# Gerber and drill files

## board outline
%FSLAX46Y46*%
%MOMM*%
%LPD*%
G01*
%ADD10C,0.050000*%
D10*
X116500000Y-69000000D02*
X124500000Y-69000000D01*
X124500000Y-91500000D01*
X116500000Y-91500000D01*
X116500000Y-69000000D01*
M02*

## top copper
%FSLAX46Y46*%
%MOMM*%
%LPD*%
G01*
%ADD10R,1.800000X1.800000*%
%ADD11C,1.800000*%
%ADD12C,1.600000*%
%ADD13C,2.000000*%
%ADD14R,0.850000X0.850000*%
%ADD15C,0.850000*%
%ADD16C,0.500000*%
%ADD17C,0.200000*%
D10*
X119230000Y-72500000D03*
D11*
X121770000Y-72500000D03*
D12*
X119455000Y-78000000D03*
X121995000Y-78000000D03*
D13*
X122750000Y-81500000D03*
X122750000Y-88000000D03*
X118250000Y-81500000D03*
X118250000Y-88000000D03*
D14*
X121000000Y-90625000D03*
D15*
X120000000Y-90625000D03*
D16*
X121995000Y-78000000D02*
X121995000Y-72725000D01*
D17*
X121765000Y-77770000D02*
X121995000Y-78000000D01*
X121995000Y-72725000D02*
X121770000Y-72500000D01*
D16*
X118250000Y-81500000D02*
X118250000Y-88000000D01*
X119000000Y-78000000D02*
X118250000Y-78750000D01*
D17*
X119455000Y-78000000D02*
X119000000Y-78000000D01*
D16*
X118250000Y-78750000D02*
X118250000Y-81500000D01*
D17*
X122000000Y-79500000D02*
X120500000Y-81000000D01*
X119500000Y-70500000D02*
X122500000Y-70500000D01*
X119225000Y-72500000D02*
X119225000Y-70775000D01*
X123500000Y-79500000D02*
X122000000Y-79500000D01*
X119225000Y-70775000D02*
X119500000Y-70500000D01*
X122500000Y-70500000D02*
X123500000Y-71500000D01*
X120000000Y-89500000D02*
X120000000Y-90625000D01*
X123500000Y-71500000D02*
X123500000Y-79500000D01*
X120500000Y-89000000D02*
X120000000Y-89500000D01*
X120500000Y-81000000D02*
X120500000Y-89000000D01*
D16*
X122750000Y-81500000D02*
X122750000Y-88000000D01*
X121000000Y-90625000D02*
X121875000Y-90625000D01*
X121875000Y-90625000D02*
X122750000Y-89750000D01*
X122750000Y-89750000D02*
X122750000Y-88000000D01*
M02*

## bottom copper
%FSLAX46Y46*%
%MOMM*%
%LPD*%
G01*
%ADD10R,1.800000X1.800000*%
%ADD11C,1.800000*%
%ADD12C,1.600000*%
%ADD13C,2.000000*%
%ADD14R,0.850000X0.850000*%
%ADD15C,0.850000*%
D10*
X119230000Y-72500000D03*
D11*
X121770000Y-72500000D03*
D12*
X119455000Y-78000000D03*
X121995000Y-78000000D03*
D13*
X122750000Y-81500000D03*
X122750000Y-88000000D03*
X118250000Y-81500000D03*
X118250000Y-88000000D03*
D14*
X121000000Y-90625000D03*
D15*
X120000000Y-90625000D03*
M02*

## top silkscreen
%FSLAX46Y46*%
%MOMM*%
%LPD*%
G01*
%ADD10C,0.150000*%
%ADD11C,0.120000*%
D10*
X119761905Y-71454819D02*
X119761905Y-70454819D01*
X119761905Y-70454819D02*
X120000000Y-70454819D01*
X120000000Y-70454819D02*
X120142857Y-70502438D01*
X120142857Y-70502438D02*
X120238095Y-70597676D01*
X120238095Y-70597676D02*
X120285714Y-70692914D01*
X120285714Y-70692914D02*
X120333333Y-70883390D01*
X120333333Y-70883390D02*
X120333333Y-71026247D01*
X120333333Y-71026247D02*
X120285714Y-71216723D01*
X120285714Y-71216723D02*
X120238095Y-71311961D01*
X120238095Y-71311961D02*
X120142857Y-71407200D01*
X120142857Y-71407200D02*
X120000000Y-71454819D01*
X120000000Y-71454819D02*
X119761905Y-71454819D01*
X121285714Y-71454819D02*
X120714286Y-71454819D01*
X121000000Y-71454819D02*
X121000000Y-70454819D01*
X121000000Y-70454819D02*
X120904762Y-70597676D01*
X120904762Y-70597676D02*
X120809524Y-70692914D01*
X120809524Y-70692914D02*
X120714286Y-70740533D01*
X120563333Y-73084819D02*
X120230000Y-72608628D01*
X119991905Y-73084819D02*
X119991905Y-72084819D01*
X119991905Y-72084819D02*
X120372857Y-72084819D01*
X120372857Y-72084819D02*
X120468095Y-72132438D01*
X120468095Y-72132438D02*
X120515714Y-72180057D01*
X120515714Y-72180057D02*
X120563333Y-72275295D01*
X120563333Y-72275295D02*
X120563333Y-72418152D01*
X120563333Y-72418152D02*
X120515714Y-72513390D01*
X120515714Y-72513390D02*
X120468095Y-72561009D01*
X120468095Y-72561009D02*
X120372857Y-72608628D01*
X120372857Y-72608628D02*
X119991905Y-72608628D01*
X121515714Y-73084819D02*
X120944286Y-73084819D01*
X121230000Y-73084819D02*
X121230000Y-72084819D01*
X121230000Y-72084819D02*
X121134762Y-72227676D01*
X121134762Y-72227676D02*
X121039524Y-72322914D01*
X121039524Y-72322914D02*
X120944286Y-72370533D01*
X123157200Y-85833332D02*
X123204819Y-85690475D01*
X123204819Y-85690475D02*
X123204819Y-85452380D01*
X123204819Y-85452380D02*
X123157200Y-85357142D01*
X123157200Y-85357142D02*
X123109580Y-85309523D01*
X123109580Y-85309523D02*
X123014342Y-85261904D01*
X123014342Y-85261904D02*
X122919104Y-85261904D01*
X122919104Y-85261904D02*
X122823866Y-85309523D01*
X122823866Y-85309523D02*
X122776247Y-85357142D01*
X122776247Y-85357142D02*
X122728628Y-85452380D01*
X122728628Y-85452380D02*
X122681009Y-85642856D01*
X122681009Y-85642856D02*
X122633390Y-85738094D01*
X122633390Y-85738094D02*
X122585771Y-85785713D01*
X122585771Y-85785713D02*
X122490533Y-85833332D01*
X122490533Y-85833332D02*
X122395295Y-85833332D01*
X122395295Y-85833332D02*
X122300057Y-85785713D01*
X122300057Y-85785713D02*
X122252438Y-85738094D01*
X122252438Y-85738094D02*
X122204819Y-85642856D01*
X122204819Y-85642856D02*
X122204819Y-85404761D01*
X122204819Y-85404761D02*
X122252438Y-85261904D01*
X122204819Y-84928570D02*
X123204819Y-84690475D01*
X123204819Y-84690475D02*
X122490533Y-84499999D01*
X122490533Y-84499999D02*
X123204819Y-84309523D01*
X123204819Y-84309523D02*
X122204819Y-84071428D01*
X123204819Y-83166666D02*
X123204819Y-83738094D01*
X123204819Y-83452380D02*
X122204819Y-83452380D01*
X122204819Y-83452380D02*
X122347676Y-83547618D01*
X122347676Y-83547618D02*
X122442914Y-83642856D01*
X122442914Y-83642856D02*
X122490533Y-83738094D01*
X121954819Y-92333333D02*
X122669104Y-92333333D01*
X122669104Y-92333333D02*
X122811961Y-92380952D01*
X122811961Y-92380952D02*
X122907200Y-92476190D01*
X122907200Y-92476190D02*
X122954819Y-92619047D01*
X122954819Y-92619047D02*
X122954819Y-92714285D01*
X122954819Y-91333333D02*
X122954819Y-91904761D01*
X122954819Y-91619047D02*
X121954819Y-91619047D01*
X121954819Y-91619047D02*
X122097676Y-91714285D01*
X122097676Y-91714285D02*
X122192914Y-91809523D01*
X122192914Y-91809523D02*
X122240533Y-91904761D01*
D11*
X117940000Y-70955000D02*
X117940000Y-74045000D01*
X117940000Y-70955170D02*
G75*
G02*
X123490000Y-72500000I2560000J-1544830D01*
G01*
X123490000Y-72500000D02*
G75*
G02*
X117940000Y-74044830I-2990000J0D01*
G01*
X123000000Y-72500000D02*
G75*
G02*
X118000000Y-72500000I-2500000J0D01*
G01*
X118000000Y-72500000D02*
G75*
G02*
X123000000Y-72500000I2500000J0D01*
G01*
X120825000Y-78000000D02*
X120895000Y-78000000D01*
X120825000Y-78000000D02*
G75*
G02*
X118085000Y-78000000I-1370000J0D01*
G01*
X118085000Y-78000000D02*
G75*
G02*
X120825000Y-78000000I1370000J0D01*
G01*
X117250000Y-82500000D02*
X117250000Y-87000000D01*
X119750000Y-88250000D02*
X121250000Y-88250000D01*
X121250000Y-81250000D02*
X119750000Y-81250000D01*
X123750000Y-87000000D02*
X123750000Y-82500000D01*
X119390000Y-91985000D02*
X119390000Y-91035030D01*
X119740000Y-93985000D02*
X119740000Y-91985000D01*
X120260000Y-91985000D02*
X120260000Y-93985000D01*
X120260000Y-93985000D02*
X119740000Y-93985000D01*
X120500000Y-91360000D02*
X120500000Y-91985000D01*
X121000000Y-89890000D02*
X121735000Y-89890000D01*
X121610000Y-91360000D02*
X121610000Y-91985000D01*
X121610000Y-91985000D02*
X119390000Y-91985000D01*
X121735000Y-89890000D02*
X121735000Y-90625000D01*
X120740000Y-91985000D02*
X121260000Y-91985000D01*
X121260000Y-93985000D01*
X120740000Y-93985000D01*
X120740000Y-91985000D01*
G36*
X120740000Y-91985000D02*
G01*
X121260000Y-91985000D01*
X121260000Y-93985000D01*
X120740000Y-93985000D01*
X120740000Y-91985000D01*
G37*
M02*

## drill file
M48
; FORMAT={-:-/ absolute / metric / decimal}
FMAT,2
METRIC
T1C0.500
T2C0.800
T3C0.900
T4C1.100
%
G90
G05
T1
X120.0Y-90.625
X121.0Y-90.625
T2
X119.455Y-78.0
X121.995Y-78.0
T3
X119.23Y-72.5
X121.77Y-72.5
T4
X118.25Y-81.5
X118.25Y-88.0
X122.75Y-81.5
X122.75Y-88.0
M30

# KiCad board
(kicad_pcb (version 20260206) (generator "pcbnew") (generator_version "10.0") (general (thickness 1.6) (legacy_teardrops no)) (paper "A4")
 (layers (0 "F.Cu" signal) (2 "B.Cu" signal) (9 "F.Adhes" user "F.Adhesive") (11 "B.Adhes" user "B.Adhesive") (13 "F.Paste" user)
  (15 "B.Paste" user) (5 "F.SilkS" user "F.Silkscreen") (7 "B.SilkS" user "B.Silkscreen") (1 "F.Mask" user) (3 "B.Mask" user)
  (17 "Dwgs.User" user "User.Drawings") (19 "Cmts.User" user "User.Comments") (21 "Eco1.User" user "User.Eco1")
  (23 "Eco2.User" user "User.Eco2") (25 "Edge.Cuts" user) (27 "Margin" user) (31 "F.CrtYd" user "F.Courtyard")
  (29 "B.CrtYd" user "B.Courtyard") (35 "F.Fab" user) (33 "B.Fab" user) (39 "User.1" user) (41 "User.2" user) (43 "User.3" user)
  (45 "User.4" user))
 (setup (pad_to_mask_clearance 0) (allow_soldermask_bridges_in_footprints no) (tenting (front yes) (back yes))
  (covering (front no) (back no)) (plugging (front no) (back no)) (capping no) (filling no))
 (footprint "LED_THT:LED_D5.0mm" (layer "F.Cu") (at 119.23 72.5)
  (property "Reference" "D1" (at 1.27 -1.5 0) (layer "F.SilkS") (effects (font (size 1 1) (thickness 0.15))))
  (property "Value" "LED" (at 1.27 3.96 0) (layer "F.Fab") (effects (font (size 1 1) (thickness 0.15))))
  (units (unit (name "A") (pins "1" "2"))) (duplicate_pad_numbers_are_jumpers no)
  (fp_line (start -1.29 -1.545) (end -1.29 1.545) (stroke (width 0.12) (type solid)) (layer "F.SilkS"))
  (fp_arc (start -1.29 -1.54483) (mid 2.071779 -2.880495) (end 4.26 0) (stroke (width 0.12) (type solid)) (layer "F.SilkS"))
  (fp_arc (start 4.26 0) (mid 2.071779 2.880495) (end -1.29 1.54483) (stroke (width 0.12) (type solid)) (layer "F.SilkS"))
  (fp_circle (center 1.27 0) (end 3.77 0) (stroke (width 0.12) (type solid)) (fill no) (layer "F.SilkS"))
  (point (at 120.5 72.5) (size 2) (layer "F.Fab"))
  (pad "1" thru_hole rect (at 0 0) (size 1.8 1.8) (drill 0.9) (layers "*.Cu" "*.Mask") (remove_unused_layers no) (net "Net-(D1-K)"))
  (pad "2" thru_hole circle (at 2.54 0) (size 1.8 1.8) (drill 0.9) (layers "*.Cu" "*.Mask") (remove_unused_layers no) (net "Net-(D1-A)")))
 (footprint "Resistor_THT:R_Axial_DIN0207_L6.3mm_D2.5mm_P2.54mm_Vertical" (layer "F.Cu") (at 119.455 78)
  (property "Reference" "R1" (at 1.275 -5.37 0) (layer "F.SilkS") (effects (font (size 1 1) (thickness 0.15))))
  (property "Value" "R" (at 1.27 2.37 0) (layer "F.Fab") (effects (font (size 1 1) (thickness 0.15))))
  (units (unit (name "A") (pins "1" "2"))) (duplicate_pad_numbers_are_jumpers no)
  (fp_line (start 1.37 0) (end 1.44 0) (stroke (width 0.12) (type solid)) (layer "F.SilkS"))
  (fp_circle (center 0 0) (end 1.37 0) (stroke (width 0.12) (type solid)) (fill no) (layer "F.SilkS"))
  (pad "1" thru_hole circle (at 0 0) (size 1.6 1.6) (drill 0.8) (layers "*.Cu" "*.Mask") (remove_unused_layers no) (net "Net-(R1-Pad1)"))
  (pad "2" thru_hole circle (at 2.54 0) (size 1.6 1.6) (drill 0.8) (layers "*.Cu" "*.Mask") (remove_unused_layers no) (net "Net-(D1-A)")))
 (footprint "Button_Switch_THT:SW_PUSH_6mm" (layer "F.Cu") (at 122.75 81.5 -90)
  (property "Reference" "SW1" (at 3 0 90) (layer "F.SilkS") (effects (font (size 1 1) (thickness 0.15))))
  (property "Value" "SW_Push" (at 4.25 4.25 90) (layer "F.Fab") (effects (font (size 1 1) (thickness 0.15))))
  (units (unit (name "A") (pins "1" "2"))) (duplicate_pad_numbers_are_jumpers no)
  (fp_line (start 1 5.5) (end 5.5 5.5) (stroke (width 0.12) (type solid)) (layer "F.SilkS"))
  (fp_line (start 6.75 3) (end 6.75 1.5) (stroke (width 0.12) (type solid)) (layer "F.SilkS"))
  (fp_line (start -0.25 1.5) (end -0.25 3) (stroke (width 0.12) (type solid)) (layer "F.SilkS"))
  (fp_line (start 5.5 -1) (end 1 -1) (stroke (width 0.12) (type solid)) (layer "F.SilkS"))
  (pad "1" thru_hole circle (at 0 0) (size 2 2) (drill 1.1) (layers "*.Cu" "*.Mask") (remove_unused_layers no) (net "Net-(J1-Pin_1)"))
  (pad "1" thru_hole circle (at 6.5 0) (size 2 2) (drill 1.1) (layers "*.Cu" "*.Mask") (remove_unused_layers no) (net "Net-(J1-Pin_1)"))
  (pad "2" thru_hole circle (at 0 4.5) (size 2 2) (drill 1.1) (layers "*.Cu" "*.Mask") (remove_unused_layers no) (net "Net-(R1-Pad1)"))
  (pad "2" thru_hole circle (at 6.5 4.5) (size 2 2) (drill 1.1) (layers "*.Cu" "*.Mask") (remove_unused_layers no) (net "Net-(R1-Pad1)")))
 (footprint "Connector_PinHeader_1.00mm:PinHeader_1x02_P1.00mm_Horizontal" (layer "F.Cu") (at 121 90.625 -90)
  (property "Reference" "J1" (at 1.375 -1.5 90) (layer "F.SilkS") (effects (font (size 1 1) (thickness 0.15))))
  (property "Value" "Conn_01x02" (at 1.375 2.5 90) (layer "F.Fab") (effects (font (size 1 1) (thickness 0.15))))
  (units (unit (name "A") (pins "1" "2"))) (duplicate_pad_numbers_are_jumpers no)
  (fp_line (start 1.36 1.61) (end 0.41003 1.61) (stroke (width 0.12) (type solid)) (layer "F.SilkS"))
  (fp_line (start 3.36 1.26) (end 1.36 1.26) (stroke (width 0.12) (type solid)) (layer "F.SilkS"))
  (fp_line (start 1.36 0.74) (end 3.36 0.74) (stroke (width 0.12) (type solid)) (layer "F.SilkS"))
  (fp_line (start 3.36 0.74) (end 3.36 1.26) (stroke (width 0.12) (type solid)) (layer "F.SilkS"))
  (fp_line (start 0.735 0.5) (end 1.36 0.5) (stroke (width 0.12) (type solid)) (layer "F.SilkS"))
  (fp_line (start -0.735 0) (end -0.735 -0.735) (stroke (width 0.12) (type solid)) (layer "F.SilkS"))
  (fp_line (start 0.735 -0.61) (end 1.36 -0.61) (stroke (width 0.12) (type solid)) (layer "F.SilkS"))
  (fp_line (start 1.36 -0.61) (end 1.36 1.61) (stroke (width 0.12) (type solid)) (layer "F.SilkS"))
  (fp_line (start -0.735 -0.735) (end 0 -0.735) (stroke (width 0.12) (type solid)) (layer "F.SilkS"))
  (fp_rect (start 1.36 -0.26) (end 3.36 0.26) (stroke (width 0.12) (type solid)) (fill yes) (layer "F.SilkS"))
  (pad "1" thru_hole rect (at 0 0 270) (size 0.85 0.85) (drill 0.5) (layers "*.Cu" "*.Mask") (remove_unused_layers no)
   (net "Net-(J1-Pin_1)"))
  (pad "2" thru_hole circle (at 0 1 270) (size 0.85 0.85) (drill 0.5) (layers "*.Cu" "*.Mask") (remove_unused_layers no) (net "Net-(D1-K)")))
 (gr_rect (start 116.5 69) (end 124.5 91.5) (stroke (width 0.05) (type default)) (fill no) (layer "Edge.Cuts"))
 (segment (start 121.995 78) (end 121.995 72.725) (width 0.5) (layer "F.Cu") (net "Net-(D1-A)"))
 (segment (start 121.765 77.77) (end 121.995 78) (width 0.2) (layer "F.Cu") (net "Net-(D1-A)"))
 (segment (start 121.995 72.725) (end 121.77 72.5) (width 0.2) (layer "F.Cu") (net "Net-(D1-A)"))
 (segment (start 118.25 81.5) (end 118.25 88) (width 0.5) (layer "F.Cu") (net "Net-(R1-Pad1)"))
 (segment (start 119 78) (end 118.25 78.75) (width 0.5) (layer "F.Cu") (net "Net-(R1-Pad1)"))
 (segment (start 119.455 78) (end 119 78) (width 0.2) (layer "F.Cu") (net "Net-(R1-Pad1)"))
 (segment (start 118.25 78.75) (end 118.25 81.5) (width 0.5) (layer "F.Cu") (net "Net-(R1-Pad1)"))
 (segment (start 122 79.5) (end 120.5 81) (width 0.2) (layer "F.Cu") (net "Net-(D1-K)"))
 (segment (start 119.5 70.5) (end 122.5 70.5) (width 0.2) (layer "F.Cu") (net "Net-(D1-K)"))
 (segment (start 119.225 72.5) (end 119.225 70.775) (width 0.2) (layer "F.Cu") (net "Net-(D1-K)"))
 (segment (start 123.5 79.5) (end 122 79.5) (width 0.2) (layer "F.Cu") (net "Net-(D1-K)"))
 (segment (start 119.225 70.775) (end 119.5 70.5) (width 0.2) (layer "F.Cu") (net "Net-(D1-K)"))
 (segment (start 122.5 70.5) (end 123.5 71.5) (width 0.2) (layer "F.Cu") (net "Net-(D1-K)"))
 (segment (start 120 89.5) (end 120 90.625) (width 0.2) (layer "F.Cu") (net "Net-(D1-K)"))
 (segment (start 123.5 71.5) (end 123.5 79.5) (width 0.2) (layer "F.Cu") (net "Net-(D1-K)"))
 (segment (start 120.5 89) (end 120 89.5) (width 0.2) (layer "F.Cu") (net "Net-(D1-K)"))
 (segment (start 120.5 81) (end 120.5 89) (width 0.2) (layer "F.Cu") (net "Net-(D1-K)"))
 (segment (start 122.75 81.5) (end 122.75 88) (width 0.5) (layer "F.Cu") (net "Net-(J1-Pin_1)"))
 (segment (start 121 90.625) (end 121.875 90.625) (width 0.5) (layer "F.Cu") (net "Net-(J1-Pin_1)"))
 (segment (start 121.875 90.625) (end 122.75 89.75) (width 0.5) (layer "F.Cu") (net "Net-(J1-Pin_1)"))
 (segment (start 122.75 89.75) (end 122.75 88) (width 0.5) (layer "F.Cu") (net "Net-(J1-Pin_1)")))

